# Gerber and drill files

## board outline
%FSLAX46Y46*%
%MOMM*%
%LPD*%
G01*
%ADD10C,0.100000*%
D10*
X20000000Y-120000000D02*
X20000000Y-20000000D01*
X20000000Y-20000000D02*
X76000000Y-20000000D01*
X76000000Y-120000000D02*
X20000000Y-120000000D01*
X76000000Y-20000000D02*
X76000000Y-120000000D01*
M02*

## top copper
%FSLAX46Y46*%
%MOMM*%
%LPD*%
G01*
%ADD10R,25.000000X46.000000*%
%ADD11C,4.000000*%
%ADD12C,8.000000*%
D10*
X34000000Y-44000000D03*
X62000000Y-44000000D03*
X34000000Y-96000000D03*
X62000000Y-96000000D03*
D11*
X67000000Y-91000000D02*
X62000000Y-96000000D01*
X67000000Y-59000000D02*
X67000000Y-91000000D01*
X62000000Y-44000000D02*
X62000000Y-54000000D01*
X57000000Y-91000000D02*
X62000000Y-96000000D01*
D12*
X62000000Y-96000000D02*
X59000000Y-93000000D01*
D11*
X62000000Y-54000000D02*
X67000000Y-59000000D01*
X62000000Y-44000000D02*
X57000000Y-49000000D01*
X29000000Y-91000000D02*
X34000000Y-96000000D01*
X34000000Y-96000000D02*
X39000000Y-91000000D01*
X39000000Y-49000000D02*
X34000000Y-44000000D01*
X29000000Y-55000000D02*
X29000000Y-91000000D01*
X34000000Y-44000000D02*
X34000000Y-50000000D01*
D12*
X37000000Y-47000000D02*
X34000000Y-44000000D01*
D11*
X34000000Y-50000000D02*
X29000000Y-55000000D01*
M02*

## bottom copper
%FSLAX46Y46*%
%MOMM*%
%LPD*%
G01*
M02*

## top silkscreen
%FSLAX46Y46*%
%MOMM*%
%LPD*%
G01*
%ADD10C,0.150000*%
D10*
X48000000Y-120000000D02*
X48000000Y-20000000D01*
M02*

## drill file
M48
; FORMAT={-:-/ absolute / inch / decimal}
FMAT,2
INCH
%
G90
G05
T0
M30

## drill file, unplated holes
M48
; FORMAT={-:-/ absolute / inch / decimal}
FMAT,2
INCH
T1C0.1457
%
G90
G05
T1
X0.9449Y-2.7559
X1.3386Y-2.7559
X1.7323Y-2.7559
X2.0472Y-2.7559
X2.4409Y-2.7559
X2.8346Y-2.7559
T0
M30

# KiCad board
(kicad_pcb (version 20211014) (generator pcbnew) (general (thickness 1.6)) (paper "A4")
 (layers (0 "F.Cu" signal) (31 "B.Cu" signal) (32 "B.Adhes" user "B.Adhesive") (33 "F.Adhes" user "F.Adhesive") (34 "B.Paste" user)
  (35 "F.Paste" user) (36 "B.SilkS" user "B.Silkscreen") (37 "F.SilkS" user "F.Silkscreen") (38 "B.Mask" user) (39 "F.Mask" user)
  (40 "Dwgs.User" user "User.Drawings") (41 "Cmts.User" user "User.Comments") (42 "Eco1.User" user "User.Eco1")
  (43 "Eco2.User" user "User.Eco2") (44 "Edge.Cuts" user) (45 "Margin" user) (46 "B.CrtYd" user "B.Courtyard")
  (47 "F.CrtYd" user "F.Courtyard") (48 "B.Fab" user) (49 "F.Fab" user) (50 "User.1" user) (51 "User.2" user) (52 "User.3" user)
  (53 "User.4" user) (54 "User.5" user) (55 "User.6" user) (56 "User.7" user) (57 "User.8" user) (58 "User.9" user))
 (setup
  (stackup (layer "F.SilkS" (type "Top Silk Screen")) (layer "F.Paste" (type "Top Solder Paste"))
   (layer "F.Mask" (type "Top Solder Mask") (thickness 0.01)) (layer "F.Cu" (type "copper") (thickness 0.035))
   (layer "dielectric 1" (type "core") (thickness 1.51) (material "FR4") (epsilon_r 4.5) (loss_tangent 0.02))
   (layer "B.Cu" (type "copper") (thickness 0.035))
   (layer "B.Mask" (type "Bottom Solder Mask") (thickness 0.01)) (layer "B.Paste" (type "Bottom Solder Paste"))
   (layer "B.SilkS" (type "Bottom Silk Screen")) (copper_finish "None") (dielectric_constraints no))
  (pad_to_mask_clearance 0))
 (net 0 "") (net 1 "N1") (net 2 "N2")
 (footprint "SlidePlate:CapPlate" (layer "F.Cu") (at 34 44)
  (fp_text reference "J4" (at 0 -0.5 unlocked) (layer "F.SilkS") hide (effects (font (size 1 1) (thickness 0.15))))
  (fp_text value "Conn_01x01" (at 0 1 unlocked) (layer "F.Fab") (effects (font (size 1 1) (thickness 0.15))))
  (pad "1" smd rect (at 0 0) (size 25 46) (layers "F.Cu") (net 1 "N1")))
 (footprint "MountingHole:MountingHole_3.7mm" (layer "F.Cu") (at 52 70)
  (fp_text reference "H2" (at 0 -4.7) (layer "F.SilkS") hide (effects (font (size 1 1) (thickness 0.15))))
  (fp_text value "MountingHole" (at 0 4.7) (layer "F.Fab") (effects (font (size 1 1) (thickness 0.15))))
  (pad "" np_thru_hole circle (at 0 0) (size 3.7 3.7) (drill 3.7) (layers *.Cu *.Mask)))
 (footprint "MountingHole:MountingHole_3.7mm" (layer "F.Cu") (at 24 70)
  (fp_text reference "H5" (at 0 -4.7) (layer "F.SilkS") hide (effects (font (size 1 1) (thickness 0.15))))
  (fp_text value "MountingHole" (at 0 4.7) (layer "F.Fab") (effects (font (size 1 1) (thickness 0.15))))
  (pad "" np_thru_hole circle (at 0 0) (size 3.7 3.7) (drill 3.7) (layers *.Cu *.Mask)))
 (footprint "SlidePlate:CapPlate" (layer "F.Cu") (at 62 44)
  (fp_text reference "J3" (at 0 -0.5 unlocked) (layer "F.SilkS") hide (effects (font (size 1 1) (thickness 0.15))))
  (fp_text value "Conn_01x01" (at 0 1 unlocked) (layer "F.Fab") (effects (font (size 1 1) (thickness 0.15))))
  (pad "1" smd rect (at 0 0) (size 25 46) (layers "F.Cu") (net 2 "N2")))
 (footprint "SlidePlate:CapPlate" (layer "F.Cu") (at 34 96)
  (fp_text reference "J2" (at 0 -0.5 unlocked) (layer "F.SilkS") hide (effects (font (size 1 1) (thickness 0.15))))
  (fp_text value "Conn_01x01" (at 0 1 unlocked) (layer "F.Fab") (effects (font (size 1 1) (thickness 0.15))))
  (pad "1" smd rect (at 0 0) (size 25 46) (layers "F.Cu") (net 1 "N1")))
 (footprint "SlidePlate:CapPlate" (layer "F.Cu") (at 62 96)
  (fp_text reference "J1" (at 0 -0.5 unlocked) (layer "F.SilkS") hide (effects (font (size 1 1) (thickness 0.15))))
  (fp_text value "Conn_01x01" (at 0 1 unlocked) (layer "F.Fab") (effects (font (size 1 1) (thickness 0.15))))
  (pad "1" smd rect (at 0 0) (size 25 46) (layers "F.Cu") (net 2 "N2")))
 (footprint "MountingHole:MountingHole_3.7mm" (layer "F.Cu") (at 72 70)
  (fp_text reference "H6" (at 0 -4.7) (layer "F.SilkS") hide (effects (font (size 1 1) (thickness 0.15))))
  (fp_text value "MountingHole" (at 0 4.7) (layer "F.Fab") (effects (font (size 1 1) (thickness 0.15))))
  (pad "" np_thru_hole circle (at 0 0) (size 3.7 3.7) (drill 3.7) (layers *.Cu *.Mask)))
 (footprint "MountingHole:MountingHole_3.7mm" (layer "F.Cu") (at 34 70)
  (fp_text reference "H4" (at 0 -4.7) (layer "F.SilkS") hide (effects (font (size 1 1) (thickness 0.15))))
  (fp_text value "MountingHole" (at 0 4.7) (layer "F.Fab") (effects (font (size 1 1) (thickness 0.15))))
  (pad "" np_thru_hole circle (at 0 0) (size 3.7 3.7) (drill 3.7) (layers *.Cu *.Mask)))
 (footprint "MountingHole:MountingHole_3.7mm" (layer "F.Cu") (at 44 70)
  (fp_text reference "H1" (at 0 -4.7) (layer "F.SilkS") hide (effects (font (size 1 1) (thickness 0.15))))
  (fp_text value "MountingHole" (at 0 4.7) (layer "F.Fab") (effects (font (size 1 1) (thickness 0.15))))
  (pad "" np_thru_hole circle (at 0 0) (size 3.7 3.7) (drill 3.7) (layers *.Cu *.Mask)))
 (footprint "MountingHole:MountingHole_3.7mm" (layer "F.Cu") (at 62 70)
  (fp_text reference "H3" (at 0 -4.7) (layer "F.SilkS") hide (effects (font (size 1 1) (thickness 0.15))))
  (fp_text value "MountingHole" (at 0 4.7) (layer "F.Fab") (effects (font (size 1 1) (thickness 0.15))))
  (pad "" np_thru_hole circle (at 0 0) (size 3.7 3.7) (drill 3.7) (layers *.Cu *.Mask)))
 (gr_line (start 48 120) (end 48 20) (layer "F.SilkS") (width 0.15))
 (gr_line (start 20 120) (end 20 20) (layer "Edge.Cuts") (width 0.1))
 (gr_line (start 20 20) (end 76 20) (layer "Edge.Cuts") (width 0.1))
 (gr_line (start 76 120) (end 20 120) (layer "Edge.Cuts") (width 0.1))
 (gr_line (start 76 20) (end 76 120) (layer "Edge.Cuts") (width 0.1))
 (segment (start 67 91) (end 62 96) (width 4) (layer "F.Cu") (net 2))
 (segment (start 67 59) (end 67 91) (width 4) (layer "F.Cu") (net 2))
 (segment (start 62 44) (end 62 54) (width 4) (layer "F.Cu") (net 2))
 (segment (start 57 91) (end 62 96) (width 4) (layer "F.Cu") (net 2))
 (segment (start 62 96) (end 59 93) (width 8) (layer "F.Cu") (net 2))
 (segment (start 62 54) (end 67 59) (width 4) (layer "F.Cu") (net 2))
 (segment (start 62 44) (end 57 49) (width 4) (layer "F.Cu") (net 2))
 (segment (start 29 91) (end 34 96) (width 4) (layer "F.Cu") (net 1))
 (segment (start 34 96) (end 39 91) (width 4) (layer "F.Cu") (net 1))
 (segment (start 39 49) (end 34 44) (width 4) (layer "F.Cu") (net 1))
 (segment (start 29 55) (end 29 91) (width 4) (layer "F.Cu") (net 1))
 (segment (start 34 44) (end 34 50) (width 4) (layer "F.Cu") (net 1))
 (segment (start 37 47) (end 34 44) (width 8) (layer "F.Cu") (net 1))
 (segment (start 34 50) (end 29 55) (width 4) (layer "F.Cu") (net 1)))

